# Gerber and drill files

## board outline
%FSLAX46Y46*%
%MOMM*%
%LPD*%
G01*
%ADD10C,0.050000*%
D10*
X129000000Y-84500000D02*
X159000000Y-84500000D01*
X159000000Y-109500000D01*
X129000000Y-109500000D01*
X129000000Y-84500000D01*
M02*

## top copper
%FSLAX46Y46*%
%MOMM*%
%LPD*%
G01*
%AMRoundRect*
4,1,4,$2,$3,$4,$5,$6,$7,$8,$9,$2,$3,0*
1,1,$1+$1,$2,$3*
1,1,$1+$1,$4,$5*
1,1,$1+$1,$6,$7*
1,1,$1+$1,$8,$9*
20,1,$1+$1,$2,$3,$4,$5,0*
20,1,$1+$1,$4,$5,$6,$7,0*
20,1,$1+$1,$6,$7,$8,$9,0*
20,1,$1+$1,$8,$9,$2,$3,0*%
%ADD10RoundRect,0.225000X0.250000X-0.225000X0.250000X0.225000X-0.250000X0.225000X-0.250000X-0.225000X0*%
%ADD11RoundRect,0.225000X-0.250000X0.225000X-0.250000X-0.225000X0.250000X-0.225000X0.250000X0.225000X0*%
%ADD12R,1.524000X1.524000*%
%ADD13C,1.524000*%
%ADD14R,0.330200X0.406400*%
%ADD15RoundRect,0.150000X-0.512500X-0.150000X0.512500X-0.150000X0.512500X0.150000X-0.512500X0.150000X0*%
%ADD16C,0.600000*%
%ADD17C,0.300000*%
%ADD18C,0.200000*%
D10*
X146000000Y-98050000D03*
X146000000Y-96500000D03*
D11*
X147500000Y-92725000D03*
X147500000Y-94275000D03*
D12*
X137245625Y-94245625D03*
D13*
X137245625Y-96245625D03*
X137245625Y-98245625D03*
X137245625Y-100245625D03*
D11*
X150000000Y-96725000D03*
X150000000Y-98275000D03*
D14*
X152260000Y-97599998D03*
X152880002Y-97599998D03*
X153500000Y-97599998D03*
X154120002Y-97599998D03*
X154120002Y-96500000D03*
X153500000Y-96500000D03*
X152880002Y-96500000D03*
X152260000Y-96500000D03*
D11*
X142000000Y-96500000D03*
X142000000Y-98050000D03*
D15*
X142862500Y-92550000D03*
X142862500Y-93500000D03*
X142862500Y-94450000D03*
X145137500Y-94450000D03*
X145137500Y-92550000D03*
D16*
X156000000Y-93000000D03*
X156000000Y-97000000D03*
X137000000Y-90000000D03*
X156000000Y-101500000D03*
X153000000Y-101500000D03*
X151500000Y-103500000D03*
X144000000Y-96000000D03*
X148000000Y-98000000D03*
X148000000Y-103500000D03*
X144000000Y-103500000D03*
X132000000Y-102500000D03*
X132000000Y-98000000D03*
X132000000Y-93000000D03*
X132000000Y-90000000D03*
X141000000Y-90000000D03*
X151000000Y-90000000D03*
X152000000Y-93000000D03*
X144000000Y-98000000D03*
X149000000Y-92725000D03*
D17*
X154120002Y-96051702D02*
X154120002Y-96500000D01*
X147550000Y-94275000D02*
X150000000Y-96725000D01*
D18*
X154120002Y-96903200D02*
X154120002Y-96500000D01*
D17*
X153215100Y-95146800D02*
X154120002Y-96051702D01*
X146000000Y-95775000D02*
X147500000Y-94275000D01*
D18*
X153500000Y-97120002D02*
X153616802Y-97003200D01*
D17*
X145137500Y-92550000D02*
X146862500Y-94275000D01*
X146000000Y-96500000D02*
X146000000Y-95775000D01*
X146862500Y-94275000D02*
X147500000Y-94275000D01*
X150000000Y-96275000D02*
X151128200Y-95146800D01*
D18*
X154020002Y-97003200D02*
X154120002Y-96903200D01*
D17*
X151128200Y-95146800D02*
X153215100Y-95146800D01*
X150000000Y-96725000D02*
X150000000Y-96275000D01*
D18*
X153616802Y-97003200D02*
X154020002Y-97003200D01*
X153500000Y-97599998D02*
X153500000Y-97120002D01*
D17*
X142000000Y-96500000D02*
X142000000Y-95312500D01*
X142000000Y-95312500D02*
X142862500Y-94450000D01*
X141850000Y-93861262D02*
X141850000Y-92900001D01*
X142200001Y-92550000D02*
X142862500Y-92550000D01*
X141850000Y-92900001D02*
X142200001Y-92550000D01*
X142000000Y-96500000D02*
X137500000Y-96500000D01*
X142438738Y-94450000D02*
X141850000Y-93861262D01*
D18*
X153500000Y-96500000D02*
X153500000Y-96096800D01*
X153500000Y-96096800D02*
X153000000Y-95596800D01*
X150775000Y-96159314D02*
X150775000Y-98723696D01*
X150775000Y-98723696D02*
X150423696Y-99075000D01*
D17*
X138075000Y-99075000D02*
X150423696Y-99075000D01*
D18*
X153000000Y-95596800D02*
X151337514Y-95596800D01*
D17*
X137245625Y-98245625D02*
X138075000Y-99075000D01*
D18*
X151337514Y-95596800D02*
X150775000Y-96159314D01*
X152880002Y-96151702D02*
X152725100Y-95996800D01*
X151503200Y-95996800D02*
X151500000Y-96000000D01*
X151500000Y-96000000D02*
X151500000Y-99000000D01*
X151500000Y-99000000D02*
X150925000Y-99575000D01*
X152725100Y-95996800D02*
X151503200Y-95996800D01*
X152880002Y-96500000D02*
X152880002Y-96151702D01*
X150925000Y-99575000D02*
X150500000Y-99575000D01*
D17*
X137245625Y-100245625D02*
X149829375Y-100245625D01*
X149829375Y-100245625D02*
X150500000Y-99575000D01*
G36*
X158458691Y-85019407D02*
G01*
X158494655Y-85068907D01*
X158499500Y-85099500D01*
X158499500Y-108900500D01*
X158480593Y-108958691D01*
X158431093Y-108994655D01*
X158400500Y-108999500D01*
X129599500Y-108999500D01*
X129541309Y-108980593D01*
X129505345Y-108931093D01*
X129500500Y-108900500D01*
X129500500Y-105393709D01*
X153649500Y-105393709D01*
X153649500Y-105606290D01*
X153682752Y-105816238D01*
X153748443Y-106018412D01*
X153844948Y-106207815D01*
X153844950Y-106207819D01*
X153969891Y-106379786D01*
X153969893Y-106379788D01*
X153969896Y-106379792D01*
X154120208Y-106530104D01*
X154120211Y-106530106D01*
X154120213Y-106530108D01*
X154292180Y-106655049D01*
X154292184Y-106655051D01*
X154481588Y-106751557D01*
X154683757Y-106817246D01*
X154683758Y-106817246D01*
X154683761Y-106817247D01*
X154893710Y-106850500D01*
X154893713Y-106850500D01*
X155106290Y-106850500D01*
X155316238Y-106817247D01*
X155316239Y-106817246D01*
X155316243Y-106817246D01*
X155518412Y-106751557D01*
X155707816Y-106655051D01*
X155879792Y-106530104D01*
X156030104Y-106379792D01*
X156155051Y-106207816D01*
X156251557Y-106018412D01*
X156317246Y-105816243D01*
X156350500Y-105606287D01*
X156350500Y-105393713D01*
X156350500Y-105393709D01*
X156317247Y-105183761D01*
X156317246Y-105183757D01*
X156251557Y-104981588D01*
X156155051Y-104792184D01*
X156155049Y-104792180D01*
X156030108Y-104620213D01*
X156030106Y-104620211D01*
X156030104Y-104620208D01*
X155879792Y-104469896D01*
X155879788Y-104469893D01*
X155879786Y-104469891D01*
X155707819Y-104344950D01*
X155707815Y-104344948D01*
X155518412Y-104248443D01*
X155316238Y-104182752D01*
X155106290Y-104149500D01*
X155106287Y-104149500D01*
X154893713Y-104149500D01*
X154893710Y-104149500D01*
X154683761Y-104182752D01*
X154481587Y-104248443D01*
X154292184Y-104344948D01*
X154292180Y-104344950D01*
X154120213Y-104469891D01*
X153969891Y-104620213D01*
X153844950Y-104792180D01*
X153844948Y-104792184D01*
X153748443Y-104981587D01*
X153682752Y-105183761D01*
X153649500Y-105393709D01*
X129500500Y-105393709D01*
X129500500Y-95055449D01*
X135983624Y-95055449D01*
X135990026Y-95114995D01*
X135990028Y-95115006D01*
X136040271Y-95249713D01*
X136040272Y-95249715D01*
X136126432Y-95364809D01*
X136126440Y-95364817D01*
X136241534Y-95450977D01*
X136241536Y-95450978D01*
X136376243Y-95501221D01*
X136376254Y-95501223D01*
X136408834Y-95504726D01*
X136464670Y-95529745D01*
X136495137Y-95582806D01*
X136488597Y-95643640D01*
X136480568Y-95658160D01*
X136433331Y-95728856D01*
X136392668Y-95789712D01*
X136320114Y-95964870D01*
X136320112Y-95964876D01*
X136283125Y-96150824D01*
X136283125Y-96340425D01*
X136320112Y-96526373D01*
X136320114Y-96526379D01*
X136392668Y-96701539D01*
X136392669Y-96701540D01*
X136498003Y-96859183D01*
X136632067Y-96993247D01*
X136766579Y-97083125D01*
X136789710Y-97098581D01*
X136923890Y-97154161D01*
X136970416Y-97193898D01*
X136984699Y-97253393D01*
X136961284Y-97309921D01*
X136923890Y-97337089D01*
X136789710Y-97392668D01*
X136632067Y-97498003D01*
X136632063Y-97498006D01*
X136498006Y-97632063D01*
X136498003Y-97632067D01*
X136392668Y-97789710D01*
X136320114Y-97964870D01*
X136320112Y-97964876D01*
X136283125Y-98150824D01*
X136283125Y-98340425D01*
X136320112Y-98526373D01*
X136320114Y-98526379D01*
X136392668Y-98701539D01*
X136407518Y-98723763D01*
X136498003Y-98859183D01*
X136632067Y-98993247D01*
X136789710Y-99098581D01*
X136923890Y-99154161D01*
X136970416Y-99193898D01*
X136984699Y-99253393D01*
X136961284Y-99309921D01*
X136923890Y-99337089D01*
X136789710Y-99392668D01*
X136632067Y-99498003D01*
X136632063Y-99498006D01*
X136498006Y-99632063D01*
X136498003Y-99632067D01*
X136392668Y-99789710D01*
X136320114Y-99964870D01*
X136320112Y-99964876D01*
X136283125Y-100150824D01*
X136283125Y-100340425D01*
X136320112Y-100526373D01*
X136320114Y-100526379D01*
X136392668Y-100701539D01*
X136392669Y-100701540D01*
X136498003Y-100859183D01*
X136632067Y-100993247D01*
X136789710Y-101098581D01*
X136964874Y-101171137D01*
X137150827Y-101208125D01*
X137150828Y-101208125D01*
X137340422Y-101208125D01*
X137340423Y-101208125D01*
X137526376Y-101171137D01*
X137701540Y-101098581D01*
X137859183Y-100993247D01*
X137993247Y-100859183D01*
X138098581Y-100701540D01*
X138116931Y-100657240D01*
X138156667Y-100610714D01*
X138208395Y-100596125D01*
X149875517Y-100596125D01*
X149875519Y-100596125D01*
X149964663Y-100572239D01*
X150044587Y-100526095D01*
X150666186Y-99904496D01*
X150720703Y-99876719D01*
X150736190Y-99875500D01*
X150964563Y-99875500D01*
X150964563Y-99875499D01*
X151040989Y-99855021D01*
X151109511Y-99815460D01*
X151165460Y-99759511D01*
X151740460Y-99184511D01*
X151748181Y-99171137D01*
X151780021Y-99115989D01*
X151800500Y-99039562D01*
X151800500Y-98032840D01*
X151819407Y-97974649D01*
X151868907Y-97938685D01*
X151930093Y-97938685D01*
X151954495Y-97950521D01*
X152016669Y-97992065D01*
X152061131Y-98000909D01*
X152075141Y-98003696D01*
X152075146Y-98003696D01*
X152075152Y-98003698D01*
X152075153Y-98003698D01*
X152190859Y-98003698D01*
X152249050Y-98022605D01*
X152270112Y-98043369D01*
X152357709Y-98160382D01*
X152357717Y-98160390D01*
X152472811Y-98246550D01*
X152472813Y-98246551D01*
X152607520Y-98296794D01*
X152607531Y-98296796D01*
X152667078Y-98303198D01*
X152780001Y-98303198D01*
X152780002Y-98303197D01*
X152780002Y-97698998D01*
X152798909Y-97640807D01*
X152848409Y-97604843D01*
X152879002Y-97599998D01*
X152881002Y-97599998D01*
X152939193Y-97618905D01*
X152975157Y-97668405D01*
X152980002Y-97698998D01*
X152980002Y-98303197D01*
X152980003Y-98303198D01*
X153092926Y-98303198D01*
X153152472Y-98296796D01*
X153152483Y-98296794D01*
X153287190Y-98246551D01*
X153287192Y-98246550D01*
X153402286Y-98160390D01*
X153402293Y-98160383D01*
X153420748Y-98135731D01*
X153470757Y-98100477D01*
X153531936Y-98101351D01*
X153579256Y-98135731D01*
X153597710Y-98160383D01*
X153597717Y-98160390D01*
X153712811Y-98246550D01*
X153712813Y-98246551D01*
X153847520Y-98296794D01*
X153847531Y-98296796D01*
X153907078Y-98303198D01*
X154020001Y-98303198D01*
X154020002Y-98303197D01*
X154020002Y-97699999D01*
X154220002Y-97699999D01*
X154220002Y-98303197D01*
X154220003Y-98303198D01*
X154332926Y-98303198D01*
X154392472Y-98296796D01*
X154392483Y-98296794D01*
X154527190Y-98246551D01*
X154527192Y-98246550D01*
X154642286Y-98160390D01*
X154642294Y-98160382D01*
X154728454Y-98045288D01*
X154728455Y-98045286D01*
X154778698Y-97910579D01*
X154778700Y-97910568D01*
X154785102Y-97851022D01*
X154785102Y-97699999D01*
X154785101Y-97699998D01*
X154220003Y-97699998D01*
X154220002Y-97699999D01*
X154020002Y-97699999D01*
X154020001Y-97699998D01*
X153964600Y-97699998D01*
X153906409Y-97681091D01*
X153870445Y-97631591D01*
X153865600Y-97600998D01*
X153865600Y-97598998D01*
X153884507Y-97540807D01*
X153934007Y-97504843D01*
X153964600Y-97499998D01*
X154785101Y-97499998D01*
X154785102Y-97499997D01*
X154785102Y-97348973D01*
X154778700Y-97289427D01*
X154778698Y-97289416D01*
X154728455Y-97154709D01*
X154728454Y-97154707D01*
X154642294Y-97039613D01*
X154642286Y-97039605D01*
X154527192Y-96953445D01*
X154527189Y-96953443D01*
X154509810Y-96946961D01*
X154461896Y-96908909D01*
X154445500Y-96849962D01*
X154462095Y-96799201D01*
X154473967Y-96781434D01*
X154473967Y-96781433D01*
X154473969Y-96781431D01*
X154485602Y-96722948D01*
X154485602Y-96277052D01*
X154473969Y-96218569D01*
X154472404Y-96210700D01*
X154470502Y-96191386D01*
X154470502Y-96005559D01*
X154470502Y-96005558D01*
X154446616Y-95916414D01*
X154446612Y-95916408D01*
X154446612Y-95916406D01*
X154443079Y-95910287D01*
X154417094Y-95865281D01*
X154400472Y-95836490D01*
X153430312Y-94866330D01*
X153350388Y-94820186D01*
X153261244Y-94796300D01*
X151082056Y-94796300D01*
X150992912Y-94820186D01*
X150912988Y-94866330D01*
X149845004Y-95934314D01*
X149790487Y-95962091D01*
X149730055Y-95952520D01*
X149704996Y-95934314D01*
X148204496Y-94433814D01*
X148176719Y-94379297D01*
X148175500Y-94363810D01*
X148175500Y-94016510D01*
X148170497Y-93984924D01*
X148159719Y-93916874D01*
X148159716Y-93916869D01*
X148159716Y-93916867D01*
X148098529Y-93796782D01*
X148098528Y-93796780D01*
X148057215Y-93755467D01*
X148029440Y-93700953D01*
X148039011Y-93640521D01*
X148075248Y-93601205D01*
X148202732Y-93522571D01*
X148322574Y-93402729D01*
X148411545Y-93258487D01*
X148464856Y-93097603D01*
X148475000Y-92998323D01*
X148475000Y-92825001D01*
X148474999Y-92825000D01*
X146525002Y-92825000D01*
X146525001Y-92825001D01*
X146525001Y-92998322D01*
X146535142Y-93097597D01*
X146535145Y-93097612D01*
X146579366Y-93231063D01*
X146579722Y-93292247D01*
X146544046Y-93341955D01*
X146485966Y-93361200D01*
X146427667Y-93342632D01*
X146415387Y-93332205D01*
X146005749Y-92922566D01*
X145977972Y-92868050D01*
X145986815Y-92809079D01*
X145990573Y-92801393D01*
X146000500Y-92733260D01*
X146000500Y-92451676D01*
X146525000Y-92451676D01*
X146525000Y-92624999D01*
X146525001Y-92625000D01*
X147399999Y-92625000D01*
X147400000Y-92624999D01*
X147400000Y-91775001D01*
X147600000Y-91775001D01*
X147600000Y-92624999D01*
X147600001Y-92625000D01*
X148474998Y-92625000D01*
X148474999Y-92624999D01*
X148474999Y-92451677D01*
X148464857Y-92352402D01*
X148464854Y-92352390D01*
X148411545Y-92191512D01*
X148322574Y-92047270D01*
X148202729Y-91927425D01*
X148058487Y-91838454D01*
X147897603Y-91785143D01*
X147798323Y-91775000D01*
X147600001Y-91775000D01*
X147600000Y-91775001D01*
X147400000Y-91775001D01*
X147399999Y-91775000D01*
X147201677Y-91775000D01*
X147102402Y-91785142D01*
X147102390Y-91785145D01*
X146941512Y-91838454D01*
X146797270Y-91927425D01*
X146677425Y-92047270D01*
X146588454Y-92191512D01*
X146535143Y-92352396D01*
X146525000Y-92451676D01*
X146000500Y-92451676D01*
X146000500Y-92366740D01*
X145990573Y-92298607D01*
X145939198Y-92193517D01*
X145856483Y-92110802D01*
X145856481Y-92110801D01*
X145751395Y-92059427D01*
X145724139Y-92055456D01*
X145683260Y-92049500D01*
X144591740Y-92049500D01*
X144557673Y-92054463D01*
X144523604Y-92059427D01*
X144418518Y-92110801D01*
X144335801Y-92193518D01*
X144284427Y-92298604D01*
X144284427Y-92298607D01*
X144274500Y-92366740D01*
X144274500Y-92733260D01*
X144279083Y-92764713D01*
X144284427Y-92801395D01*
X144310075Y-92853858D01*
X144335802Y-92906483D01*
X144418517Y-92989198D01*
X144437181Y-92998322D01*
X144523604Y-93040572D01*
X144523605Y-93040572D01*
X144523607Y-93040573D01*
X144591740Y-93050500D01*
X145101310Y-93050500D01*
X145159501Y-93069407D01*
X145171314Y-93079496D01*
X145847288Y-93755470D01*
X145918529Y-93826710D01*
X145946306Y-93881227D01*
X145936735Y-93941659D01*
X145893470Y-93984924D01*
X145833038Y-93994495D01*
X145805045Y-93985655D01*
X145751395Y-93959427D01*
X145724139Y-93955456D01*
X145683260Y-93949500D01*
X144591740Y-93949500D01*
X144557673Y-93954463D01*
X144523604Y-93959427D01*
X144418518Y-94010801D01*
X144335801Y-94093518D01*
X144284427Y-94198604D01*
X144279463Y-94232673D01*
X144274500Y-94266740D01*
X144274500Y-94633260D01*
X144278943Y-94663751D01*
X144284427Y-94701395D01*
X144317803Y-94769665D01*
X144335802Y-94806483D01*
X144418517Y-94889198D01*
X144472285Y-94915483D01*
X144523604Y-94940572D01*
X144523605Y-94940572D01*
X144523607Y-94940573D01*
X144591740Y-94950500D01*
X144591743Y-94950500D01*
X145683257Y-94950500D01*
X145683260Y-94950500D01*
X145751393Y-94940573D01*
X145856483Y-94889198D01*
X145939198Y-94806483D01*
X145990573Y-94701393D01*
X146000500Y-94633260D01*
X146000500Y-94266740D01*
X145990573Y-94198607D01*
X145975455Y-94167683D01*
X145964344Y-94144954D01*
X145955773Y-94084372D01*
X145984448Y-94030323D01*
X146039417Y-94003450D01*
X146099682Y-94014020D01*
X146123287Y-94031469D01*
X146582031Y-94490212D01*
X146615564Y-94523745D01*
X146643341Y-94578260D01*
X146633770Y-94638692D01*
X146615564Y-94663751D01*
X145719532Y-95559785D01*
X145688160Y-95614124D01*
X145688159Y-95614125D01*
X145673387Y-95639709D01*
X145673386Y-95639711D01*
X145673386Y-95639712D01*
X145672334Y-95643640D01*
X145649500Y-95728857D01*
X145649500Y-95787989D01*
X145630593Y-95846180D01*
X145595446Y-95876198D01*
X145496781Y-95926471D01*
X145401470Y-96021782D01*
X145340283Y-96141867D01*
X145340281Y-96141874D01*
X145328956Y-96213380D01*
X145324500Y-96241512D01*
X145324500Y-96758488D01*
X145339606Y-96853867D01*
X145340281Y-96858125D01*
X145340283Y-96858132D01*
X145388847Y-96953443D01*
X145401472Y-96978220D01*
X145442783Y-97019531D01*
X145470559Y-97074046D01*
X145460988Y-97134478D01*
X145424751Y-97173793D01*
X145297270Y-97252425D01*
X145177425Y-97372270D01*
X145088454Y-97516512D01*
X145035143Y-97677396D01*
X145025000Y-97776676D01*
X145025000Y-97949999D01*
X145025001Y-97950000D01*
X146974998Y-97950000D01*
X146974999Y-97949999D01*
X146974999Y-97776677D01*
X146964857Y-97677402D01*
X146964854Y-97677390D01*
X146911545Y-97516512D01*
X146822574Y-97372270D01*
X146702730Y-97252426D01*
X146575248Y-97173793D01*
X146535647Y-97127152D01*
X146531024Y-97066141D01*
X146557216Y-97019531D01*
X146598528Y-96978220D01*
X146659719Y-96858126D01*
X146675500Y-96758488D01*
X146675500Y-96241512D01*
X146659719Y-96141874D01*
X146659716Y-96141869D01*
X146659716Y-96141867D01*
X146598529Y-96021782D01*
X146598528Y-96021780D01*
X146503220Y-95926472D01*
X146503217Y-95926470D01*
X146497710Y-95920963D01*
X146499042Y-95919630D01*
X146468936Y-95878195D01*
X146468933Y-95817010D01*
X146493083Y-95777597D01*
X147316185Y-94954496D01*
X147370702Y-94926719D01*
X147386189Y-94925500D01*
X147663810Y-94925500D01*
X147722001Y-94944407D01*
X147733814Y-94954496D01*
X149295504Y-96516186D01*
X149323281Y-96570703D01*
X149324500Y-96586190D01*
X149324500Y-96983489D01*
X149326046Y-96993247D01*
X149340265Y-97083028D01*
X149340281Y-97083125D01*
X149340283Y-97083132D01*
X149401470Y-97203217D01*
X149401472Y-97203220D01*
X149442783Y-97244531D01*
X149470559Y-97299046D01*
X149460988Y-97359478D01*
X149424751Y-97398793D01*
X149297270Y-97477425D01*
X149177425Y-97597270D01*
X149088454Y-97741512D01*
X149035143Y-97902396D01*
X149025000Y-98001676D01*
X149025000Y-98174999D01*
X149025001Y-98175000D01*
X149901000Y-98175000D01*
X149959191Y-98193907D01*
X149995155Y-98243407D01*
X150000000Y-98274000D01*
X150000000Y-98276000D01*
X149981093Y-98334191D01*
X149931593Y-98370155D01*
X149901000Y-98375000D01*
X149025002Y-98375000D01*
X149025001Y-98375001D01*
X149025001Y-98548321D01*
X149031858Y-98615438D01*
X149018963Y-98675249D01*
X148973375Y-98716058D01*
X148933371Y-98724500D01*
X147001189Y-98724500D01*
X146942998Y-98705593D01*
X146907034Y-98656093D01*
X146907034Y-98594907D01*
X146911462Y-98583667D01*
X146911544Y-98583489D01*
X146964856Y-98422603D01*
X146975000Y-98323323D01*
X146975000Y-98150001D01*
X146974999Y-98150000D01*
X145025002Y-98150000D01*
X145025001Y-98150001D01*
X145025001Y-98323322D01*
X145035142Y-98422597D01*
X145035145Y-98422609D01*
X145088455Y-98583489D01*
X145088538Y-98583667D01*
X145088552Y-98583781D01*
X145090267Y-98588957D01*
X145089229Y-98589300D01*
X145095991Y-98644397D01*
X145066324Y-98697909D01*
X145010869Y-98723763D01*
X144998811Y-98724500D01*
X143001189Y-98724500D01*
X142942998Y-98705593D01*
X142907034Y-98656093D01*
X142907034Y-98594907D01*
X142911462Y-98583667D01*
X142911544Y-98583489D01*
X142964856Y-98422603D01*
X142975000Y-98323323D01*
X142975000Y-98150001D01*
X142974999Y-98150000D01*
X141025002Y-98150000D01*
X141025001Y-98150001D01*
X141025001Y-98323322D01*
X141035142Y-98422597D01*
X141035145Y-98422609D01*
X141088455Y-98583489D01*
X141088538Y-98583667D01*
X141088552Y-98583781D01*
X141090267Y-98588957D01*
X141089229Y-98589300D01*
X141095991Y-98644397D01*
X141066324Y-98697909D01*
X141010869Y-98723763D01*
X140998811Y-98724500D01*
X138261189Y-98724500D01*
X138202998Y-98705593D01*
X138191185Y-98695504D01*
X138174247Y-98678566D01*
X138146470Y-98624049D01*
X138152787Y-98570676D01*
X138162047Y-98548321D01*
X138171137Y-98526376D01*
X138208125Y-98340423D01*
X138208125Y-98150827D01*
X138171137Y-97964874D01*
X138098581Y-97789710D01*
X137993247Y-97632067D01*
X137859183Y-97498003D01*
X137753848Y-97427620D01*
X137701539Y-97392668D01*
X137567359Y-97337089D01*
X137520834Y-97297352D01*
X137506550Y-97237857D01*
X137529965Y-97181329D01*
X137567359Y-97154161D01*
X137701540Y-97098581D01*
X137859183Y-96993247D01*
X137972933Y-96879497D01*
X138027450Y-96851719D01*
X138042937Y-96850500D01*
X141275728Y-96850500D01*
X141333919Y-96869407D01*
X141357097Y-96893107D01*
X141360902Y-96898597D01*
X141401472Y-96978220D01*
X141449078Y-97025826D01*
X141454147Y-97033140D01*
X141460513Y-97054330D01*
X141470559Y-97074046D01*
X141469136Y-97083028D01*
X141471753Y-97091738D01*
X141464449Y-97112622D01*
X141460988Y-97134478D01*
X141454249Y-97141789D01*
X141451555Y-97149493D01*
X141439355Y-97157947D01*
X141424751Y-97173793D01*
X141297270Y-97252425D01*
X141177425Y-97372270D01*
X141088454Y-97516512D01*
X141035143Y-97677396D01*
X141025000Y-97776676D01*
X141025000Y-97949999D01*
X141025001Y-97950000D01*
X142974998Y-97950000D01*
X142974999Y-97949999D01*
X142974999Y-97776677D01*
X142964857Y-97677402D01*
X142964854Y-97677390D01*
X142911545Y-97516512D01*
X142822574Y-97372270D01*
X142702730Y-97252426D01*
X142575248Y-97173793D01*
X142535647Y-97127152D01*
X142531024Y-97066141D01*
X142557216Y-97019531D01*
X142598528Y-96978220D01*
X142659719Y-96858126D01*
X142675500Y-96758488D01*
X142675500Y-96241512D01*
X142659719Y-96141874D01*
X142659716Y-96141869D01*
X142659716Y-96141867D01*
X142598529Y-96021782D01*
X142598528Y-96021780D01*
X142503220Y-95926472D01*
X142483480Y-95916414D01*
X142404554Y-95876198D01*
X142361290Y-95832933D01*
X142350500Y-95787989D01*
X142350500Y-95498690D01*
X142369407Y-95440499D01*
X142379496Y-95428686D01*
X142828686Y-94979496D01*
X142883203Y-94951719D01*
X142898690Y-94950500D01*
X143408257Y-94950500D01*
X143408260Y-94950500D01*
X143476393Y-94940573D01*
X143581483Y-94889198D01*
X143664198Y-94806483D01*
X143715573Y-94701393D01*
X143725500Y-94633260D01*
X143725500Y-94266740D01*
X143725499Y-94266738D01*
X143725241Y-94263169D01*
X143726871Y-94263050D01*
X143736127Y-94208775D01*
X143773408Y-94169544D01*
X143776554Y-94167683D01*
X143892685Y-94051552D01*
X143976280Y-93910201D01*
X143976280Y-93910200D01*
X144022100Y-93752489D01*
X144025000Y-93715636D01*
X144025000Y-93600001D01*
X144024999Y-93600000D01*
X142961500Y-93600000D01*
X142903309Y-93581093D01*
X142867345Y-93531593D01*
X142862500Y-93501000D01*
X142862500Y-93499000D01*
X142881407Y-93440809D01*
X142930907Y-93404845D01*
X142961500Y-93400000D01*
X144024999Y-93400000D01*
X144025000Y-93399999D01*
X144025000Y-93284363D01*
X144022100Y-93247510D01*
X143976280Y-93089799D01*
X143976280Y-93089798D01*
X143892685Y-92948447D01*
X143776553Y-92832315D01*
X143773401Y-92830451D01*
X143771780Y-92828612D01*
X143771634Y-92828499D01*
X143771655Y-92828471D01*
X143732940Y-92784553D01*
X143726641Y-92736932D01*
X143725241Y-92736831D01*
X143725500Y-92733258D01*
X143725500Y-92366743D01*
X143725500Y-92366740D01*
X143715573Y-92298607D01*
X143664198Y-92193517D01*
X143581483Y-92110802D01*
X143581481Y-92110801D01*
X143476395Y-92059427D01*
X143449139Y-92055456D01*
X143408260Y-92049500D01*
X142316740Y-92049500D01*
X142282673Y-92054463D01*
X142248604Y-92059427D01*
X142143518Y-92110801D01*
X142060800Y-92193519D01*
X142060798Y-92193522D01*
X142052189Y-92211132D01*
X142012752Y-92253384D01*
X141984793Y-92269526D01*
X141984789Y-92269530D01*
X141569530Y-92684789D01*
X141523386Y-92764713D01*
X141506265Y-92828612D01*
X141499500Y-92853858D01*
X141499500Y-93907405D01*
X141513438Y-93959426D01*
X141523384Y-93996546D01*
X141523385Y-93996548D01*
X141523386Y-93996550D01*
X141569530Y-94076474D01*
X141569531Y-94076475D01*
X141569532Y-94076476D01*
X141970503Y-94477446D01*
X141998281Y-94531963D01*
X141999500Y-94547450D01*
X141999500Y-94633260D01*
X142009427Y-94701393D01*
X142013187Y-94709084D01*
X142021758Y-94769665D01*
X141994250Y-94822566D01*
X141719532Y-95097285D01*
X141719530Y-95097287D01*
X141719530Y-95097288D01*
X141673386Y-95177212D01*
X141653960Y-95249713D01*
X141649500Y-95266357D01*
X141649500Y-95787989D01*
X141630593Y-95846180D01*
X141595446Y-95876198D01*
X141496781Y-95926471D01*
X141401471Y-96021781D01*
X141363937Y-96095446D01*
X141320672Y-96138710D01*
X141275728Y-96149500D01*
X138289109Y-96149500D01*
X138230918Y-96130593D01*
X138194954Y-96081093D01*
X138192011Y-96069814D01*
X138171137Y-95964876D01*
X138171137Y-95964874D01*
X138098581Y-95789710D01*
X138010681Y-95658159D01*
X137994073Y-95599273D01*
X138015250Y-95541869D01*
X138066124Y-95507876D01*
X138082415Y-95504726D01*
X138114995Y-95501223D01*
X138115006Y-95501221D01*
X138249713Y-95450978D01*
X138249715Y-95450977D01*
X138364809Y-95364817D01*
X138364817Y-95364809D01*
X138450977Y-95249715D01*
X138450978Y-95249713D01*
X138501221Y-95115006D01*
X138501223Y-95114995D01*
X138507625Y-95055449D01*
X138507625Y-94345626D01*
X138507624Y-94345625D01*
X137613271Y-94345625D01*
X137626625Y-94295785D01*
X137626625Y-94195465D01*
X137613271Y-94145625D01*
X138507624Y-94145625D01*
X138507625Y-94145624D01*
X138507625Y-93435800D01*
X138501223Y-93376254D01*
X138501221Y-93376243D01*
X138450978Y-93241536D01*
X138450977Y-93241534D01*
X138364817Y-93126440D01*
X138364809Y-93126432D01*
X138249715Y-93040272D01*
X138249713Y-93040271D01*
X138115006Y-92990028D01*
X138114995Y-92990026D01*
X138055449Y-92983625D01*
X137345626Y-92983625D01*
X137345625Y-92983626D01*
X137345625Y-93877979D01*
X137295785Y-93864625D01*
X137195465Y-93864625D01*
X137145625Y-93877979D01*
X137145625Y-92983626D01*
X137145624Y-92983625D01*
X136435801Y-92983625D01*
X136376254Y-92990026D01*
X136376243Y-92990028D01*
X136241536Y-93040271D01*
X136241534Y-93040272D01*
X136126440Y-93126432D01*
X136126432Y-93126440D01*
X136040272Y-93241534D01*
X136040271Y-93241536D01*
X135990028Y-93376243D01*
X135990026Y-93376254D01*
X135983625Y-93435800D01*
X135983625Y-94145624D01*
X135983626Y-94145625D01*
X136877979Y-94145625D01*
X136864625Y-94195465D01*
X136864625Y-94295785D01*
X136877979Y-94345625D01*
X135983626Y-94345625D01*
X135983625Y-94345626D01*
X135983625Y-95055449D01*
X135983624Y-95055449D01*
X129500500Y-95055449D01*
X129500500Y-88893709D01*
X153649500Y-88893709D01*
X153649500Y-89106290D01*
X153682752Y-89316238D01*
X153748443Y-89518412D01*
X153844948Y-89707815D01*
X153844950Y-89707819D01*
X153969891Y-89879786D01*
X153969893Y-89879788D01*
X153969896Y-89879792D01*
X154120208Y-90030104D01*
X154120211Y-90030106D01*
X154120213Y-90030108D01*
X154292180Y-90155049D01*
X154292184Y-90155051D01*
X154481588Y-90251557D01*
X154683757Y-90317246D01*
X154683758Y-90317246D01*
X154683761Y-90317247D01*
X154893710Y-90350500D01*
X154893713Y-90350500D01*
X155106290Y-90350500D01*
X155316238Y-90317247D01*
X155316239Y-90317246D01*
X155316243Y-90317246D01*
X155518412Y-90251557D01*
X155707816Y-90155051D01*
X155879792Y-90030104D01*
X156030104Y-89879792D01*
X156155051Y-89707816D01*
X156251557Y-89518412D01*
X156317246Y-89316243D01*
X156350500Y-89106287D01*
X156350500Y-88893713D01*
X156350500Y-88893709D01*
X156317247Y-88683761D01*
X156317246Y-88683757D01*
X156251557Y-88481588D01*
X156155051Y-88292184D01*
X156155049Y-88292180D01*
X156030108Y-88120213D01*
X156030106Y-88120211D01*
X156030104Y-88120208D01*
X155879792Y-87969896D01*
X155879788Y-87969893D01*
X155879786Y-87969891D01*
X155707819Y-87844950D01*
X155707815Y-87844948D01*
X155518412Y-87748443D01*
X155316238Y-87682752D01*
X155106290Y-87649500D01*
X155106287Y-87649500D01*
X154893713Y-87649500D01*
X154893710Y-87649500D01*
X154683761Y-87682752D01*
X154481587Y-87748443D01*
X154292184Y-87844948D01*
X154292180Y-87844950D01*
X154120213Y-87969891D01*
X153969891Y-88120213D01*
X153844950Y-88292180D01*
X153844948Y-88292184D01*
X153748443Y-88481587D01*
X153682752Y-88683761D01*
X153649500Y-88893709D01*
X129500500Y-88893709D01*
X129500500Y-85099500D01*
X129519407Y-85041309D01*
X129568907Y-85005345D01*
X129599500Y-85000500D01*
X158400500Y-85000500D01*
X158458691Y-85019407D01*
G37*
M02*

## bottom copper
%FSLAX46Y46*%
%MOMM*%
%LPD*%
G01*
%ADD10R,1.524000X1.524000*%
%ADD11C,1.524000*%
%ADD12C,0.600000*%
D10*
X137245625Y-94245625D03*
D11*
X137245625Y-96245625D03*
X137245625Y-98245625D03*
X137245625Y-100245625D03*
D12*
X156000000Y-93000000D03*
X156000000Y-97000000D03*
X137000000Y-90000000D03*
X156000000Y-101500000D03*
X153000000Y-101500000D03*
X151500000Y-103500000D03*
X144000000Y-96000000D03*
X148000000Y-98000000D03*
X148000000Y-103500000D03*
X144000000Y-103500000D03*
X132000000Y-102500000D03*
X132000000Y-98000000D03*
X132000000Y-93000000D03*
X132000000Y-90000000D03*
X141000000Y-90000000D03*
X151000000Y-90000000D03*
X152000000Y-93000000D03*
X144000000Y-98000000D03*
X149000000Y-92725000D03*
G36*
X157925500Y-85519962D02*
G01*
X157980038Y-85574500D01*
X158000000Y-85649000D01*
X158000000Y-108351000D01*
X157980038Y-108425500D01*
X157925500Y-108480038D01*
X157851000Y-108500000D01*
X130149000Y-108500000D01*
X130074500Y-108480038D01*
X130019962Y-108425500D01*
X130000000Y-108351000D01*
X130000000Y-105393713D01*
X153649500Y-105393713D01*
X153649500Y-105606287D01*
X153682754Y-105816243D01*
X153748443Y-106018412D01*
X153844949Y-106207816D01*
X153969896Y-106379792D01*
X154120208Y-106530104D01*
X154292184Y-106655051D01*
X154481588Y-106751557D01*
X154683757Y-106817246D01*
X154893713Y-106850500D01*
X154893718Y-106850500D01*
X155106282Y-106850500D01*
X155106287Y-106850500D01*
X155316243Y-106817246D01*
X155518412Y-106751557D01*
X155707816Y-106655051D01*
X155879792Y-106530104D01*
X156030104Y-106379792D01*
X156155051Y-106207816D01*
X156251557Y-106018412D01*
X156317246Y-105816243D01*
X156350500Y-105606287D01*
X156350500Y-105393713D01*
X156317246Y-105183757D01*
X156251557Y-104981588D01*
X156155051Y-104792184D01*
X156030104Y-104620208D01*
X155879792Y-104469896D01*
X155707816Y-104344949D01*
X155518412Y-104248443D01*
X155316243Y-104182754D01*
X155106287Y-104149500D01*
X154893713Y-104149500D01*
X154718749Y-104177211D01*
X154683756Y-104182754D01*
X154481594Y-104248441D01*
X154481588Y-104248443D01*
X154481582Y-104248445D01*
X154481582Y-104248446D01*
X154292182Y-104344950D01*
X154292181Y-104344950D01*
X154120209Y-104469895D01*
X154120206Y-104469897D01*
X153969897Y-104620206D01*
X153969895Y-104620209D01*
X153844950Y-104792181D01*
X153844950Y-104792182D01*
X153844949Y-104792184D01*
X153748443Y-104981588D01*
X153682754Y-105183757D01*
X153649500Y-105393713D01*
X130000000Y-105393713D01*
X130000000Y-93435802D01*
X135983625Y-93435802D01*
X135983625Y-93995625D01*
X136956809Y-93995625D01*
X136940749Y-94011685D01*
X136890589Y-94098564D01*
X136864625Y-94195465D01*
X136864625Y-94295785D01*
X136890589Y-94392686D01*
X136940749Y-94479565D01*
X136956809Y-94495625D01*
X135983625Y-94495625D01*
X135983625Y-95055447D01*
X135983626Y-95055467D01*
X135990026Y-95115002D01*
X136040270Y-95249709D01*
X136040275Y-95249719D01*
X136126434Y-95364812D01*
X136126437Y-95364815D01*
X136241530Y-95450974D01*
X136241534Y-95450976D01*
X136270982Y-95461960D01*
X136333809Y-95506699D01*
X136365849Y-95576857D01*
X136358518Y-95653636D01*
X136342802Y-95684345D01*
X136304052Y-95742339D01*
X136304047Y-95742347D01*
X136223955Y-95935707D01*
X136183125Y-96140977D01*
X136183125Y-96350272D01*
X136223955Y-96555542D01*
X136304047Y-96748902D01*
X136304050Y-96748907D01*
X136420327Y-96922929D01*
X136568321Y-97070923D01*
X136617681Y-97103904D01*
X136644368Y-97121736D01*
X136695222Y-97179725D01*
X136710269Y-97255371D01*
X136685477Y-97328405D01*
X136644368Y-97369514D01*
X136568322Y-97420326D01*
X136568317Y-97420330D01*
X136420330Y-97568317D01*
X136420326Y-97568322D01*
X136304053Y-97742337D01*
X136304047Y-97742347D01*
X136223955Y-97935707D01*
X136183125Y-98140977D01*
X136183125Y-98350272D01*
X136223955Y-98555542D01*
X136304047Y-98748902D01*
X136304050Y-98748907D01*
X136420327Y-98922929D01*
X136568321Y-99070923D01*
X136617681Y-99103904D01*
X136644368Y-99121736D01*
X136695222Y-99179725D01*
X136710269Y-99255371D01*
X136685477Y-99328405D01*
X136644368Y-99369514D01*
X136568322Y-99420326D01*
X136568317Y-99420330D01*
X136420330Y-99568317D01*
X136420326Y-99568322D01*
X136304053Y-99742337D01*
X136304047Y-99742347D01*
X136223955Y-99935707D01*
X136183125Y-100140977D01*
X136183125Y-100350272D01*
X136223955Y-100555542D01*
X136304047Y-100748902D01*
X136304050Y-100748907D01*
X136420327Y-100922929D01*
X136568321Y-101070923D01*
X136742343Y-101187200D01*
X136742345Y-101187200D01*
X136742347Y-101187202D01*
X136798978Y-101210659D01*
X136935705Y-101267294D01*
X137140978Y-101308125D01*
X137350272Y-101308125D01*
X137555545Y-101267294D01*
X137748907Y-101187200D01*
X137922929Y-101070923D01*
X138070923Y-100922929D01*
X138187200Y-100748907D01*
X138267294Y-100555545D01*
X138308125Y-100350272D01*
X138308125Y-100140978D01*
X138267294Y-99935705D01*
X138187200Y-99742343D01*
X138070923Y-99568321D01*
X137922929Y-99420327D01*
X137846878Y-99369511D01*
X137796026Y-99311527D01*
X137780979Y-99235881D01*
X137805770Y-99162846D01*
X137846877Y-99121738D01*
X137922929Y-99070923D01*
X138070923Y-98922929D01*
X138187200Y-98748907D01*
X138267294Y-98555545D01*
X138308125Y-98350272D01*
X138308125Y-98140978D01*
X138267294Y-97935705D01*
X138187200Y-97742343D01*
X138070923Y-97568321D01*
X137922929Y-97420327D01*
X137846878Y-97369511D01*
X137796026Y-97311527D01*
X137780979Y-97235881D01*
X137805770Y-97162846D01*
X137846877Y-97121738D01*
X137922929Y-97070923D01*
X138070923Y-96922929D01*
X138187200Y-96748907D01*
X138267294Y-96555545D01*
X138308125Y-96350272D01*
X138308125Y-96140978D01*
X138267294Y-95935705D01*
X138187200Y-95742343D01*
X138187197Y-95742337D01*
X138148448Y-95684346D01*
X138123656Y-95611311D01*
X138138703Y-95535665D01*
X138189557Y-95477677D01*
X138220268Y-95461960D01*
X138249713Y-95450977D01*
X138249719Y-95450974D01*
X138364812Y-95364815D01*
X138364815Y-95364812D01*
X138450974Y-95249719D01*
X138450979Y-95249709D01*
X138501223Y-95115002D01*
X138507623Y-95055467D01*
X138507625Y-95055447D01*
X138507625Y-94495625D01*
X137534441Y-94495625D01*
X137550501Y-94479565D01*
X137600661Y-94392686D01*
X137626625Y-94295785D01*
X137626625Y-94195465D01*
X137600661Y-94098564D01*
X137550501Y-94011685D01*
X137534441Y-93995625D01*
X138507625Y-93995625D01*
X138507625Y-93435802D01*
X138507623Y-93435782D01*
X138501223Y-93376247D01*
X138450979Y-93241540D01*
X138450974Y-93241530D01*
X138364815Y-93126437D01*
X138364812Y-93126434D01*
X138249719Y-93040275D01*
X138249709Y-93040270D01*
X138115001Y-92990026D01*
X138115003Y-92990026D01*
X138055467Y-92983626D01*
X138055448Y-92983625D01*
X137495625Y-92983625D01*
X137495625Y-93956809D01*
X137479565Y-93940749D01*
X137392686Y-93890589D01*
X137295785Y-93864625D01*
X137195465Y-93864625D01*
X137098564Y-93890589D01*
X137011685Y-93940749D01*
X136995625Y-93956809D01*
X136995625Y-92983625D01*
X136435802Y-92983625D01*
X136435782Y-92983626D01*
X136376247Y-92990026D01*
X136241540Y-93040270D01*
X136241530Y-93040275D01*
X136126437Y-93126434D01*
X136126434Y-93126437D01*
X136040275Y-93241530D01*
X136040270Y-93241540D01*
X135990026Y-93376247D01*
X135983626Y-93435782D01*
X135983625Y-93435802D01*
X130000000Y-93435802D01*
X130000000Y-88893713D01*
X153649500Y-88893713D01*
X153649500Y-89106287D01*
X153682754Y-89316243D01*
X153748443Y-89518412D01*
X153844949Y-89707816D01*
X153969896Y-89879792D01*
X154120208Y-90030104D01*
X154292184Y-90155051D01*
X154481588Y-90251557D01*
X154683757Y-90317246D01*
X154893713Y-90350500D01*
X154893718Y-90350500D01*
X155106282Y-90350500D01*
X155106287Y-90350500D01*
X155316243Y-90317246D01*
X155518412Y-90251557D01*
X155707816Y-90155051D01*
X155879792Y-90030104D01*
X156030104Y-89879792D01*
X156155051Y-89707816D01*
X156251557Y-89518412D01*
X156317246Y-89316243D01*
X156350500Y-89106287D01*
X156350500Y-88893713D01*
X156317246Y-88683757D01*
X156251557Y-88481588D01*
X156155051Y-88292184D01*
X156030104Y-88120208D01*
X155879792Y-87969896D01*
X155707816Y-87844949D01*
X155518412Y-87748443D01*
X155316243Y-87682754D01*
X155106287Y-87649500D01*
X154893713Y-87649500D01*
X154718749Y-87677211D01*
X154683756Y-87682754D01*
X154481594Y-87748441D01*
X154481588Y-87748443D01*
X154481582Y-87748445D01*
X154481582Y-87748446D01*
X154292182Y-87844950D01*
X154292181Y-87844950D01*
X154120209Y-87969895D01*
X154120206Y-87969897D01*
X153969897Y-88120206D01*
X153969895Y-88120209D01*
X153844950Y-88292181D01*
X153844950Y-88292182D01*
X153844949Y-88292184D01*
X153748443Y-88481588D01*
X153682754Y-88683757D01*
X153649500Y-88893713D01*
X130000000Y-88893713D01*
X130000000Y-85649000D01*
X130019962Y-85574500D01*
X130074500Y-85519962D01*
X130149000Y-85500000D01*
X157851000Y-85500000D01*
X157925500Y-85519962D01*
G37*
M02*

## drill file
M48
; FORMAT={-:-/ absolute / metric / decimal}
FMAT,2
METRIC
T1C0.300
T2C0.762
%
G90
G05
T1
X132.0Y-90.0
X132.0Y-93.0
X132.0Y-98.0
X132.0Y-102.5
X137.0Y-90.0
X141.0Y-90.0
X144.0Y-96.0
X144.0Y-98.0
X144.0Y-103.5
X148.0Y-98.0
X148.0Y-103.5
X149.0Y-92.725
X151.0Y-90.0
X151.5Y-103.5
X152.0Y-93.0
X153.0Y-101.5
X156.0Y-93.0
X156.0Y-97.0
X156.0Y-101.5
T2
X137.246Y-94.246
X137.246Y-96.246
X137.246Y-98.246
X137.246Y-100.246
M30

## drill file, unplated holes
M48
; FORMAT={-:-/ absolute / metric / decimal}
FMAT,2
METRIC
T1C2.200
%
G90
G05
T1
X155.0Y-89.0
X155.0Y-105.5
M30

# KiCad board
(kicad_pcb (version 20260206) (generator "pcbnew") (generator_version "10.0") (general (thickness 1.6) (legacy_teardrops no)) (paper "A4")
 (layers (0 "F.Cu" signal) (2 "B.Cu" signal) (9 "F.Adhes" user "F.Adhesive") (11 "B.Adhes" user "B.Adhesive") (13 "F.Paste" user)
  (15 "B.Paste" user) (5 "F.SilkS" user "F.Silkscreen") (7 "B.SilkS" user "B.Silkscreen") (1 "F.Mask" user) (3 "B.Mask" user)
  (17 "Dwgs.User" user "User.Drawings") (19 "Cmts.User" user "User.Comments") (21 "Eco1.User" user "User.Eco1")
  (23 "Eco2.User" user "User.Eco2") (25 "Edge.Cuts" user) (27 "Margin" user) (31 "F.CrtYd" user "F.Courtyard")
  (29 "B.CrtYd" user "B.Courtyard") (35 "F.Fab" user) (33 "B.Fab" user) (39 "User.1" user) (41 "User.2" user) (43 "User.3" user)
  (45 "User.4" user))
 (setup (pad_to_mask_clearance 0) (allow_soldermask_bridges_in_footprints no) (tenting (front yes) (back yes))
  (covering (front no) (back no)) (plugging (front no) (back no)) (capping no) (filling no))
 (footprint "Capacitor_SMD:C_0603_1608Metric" (layer "F.Cu") (at 146 97.275 90)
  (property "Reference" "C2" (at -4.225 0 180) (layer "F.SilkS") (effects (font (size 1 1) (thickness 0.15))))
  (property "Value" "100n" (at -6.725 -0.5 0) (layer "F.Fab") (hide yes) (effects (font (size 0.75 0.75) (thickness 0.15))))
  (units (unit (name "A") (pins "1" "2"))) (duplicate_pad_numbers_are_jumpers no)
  (pad "1" smd roundrect (at -0.775 0 90) (size 0.9 0.95) (layers "F.Cu" "F.Mask" "F.Paste") (roundrect_rratio 0.25) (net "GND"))
  (pad "2" smd roundrect (at 0.775 0 90) (size 0.9 0.95) (layers "F.Cu" "F.Mask" "F.Paste") (roundrect_rratio 0.25) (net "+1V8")))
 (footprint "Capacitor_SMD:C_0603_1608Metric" (layer "F.Cu") (at 147.5 93.5 -90)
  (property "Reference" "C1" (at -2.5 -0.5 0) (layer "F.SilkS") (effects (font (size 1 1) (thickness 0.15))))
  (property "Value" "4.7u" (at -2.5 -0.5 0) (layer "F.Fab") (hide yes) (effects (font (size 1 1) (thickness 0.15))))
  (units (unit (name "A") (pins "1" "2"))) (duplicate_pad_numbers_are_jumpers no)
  (pad "1" smd roundrect (at -0.775 0 270) (size 0.9 0.95) (layers "F.Cu" "F.Mask" "F.Paste") (roundrect_rratio 0.25) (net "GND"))
  (pad "2" smd roundrect (at 0.775 0 270) (size 0.9 0.95) (layers "F.Cu" "F.Mask" "F.Paste") (roundrect_rratio 0.25) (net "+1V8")))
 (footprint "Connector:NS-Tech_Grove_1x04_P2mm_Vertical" (layer "F.Cu") (at 137.245625 94.245625)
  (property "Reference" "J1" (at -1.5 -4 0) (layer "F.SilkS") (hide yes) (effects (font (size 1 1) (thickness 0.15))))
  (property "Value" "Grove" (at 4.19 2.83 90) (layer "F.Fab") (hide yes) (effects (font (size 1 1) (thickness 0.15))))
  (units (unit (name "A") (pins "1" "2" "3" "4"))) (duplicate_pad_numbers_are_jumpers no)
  (pad "1" thru_hole rect (at 0 0) (size 1.524 1.524) (drill 0.762) (layers "*.Cu" "*.Mask") (remove_unused_layers no) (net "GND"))
  (pad "2" thru_hole circle (at 0 2) (size 1.524 1.524) (drill 0.762) (layers "*.Cu" "*.Mask") (remove_unused_layers no) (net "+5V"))
  (pad "3" thru_hole circle (at 0 4) (size 1.524 1.524) (drill 0.762) (layers "*.Cu" "*.Mask") (remove_unused_layers no) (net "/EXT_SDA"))
  (pad "4" thru_hole circle (at 0 6) (size 1.524 1.524) (drill 0.762) (layers "*.Cu" "*.Mask") (remove_unused_layers no) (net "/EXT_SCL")))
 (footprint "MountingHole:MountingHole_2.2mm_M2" (layer "F.Cu") (at 155 105.5)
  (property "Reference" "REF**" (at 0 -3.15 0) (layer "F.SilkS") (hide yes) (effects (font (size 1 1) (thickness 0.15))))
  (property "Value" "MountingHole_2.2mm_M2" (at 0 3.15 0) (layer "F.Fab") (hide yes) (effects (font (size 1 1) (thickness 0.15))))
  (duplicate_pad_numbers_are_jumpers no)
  (pad "" np_thru_hole circle (at 0 0) (size 2.2 2.2) (drill 2.2) (layers "*.Cu" "*.Mask")))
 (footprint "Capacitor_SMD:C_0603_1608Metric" (layer "F.Cu") (at 150 97.5 -90)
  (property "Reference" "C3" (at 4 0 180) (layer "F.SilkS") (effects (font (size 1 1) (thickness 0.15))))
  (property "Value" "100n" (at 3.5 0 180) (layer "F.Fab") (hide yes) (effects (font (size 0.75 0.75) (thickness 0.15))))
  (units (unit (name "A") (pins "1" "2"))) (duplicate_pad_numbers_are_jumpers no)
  (pad "1" smd roundrect (at -0.775 0 270) (size 0.9 0.95) (layers "F.Cu" "F.Mask" "F.Paste") (roundrect_rratio 0.25) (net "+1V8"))
  (pad "2" smd roundrect (at 0.775 0 270) (size 0.9 0.95) (layers "F.Cu" "F.Mask" "F.Paste") (roundrect_rratio 0.25) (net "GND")))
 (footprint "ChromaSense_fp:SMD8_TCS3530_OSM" (layer "F.Cu") (at 153.190001 97.049999 90)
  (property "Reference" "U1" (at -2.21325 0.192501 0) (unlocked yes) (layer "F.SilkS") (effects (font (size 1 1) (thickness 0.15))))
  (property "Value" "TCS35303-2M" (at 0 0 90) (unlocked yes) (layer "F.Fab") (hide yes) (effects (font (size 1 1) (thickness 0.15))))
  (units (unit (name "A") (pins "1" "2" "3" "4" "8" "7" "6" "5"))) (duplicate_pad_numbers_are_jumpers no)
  (pad "1" smd rect (at -0.549999 -0.930001 90) (size 0.4064 0.3302) (layers "F.Cu" "F.Mask" "F.Paste") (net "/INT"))
  (pad "2" smd rect (at -0.549999 -0.309999 90) (size 0.4064 0.3302) (layers "F.Cu" "F.Mask" "F.Paste") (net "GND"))
  (pad "3" smd rect (at -0.549999 0.309999 90) (size 0.4064 0.3302) (layers "F.Cu" "F.Mask" "F.Paste") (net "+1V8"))
  (pad "4" smd rect (at -0.549999 0.930001 90) (size 0.4064 0.3302) (layers "F.Cu" "F.Mask" "F.Paste") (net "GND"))
  (pad "5" smd rect (at 0.549999 0.930001 90) (size 0.4064 0.3302) (layers "F.Cu" "F.Mask" "F.Paste") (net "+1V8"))
  (pad "6" smd rect (at 0.549999 0.309999 90) (size 0.4064 0.3302) (layers "F.Cu" "F.Mask" "F.Paste") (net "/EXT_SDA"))
  (pad "7" smd rect (at 0.549999 -0.309999 90) (size 0.4064 0.3302) (layers "F.Cu" "F.Mask" "F.Paste") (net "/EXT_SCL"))
  (pad "8" smd rect (at 0.549999 -0.930001 90) (size 0.4064 0.3302) (layers "F.Cu" "F.Mask" "F.Paste")
   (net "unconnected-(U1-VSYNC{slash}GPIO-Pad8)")))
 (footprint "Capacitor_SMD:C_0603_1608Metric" (layer "F.Cu") (at 142 97.275 -90)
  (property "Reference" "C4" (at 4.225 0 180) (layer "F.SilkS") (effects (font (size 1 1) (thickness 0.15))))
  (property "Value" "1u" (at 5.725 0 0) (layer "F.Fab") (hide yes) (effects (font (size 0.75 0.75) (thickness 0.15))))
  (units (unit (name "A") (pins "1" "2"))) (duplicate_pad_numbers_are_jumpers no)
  (pad "1" smd roundrect (at -0.775 0 270) (size 0.9 0.95) (layers "F.Cu" "F.Mask" "F.Paste") (roundrect_rratio 0.25) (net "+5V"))
  (pad "2" smd roundrect (at 0.775 0 270) (size 0.9 0.95) (layers "F.Cu" "F.Mask" "F.Paste") (roundrect_rratio 0.25) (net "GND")))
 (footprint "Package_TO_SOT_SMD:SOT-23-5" (layer "F.Cu") (at 144 93.5)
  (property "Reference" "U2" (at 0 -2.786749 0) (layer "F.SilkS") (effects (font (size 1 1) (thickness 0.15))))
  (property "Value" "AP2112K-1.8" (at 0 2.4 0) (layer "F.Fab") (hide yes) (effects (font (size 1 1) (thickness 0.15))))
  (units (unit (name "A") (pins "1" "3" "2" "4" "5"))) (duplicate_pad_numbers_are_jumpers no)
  (pad "1" smd roundrect (at -1.1375 -0.95) (size 1.325 0.6) (layers "F.Cu" "F.Mask" "F.Paste") (roundrect_rratio 0.25) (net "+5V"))
  (pad "2" smd roundrect (at -1.1375 0) (size 1.325 0.6) (layers "F.Cu" "F.Mask" "F.Paste") (roundrect_rratio 0.25) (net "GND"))
  (pad "3" smd roundrect (at -1.1375 0.95) (size 1.325 0.6) (layers "F.Cu" "F.Mask" "F.Paste") (roundrect_rratio 0.25) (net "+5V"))
  (pad "4" smd roundrect (at 1.1375 0.95) (size 1.325 0.6) (layers "F.Cu" "F.Mask" "F.Paste") (roundrect_rratio 0.25)
   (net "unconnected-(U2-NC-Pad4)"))
  (pad "5" smd roundrect (at 1.1375 -0.95) (size 1.325 0.6) (layers "F.Cu" "F.Mask" "F.Paste") (roundrect_rratio 0.25) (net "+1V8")))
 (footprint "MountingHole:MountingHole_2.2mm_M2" (layer "F.Cu") (at 155 89)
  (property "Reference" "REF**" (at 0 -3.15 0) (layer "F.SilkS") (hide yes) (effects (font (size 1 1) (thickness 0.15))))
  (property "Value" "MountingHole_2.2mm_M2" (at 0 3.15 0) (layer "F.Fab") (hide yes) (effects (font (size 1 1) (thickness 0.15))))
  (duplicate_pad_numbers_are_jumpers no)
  (pad "" np_thru_hole circle (at 0 0) (size 2.2 2.2) (drill 2.2) (layers "*.Cu" "*.Mask")))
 (gr_rect (start 129 84.5) (end 159 109.5) (stroke (width 0.05) (type solid)) (fill no) (layer "Edge.Cuts"))
 (via (at 156 93) (size 0.6) (drill 0.3) (layers "F.Cu" "B.Cu") (free yes) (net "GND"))
 (via (at 144 96) (size 0.6) (drill 0.3) (layers "F.Cu" "B.Cu") (free yes) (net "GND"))
 (via (at 151 90) (size 0.6) (drill 0.3) (layers "F.Cu" "B.Cu") (free yes) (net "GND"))
 (via (at 152 93) (size 0.6) (drill 0.3) (layers "F.Cu" "B.Cu") (free yes) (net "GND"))
 (via (at 148 98) (size 0.6) (drill 0.3) (layers "F.Cu" "B.Cu") (free yes) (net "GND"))
 (via (at 156 101.5) (size 0.6) (drill 0.3) (layers "F.Cu" "B.Cu") (free yes) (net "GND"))
 (via (at 148 103.5) (size 0.6) (drill 0.3) (layers "F.Cu" "B.Cu") (free yes) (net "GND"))
 (via (at 132 90) (size 0.6) (drill 0.3) (layers "F.Cu" "B.Cu") (free yes) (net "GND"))
 (via (at 132 102.5) (size 0.6) (drill 0.3) (layers "F.Cu" "B.Cu") (free yes) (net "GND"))
 (via (at 153 101.5) (size 0.6) (drill 0.3) (layers "F.Cu" "B.Cu") (free yes) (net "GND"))
 (via (at 132 93) (size 0.6) (drill 0.3) (layers "F.Cu" "B.Cu") (free yes) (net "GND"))
 (via (at 144 98) (size 0.6) (drill 0.3) (layers "F.Cu" "B.Cu") (free yes) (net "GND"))
 (via (at 141 90) (size 0.6) (drill 0.3) (layers "F.Cu" "B.Cu") (free yes) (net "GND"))
 (via (at 151.5 103.5) (size 0.6) (drill 0.3) (layers "F.Cu" "B.Cu") (free yes) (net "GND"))
 (via (at 149 92.725) (size 0.6) (drill 0.3) (layers "F.Cu" "B.Cu") (free yes) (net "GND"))
 (via (at 144 103.5) (size 0.6) (drill 0.3) (layers "F.Cu" "B.Cu") (free yes) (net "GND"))
 (via (at 137 90) (size 0.6) (drill 0.3) (layers "F.Cu" "B.Cu") (free yes) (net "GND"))
 (via (at 132 98) (size 0.6) (drill 0.3) (layers "F.Cu" "B.Cu") (free yes) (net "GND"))
 (via (at 156 97) (size 0.6) (drill 0.3) (layers "F.Cu" "B.Cu") (free yes) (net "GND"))
 (segment (start 154.120002 96.051702) (end 154.120002 96.5) (width 0.3) (layer "F.Cu") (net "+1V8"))
 (segment (start 147.55 94.275) (end 150 96.725) (width 0.3) (layer "F.Cu") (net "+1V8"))
 (segment (start 154.120002 96.9032) (end 154.120002 96.5) (width 0.2) (layer "F.Cu") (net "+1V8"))
 (segment (start 153.2151 95.1468) (end 154.120002 96.051702) (width 0.3) (layer "F.Cu") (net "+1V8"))
 (segment (start 146 95.775) (end 147.5 94.275) (width 0.3) (layer "F.Cu") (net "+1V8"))
 (segment (start 153.5 97.120002) (end 153.616802 97.0032) (width 0.2) (layer "F.Cu") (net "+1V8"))
 (segment (start 145.1375 92.55) (end 146.8625 94.275) (width 0.3) (layer "F.Cu") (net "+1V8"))
 (segment (start 146 96.5) (end 146 95.775) (width 0.3) (layer "F.Cu") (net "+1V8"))
 (segment (start 146.8625 94.275) (end 147.5 94.275) (width 0.3) (layer "F.Cu") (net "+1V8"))
 (segment (start 150 96.275) (end 151.1282 95.1468) (width 0.3) (layer "F.Cu") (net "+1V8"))
 (segment (start 154.020002 97.0032) (end 154.120002 96.9032) (width 0.2) (layer "F.Cu") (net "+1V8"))
 (segment (start 151.1282 95.1468) (end 153.2151 95.1468) (width 0.3) (layer "F.Cu") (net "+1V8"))
 (segment (start 150 96.725) (end 150 96.275) (width 0.3) (layer "F.Cu") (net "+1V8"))
 (segment (start 153.616802 97.0032) (end 154.020002 97.0032) (width 0.2) (layer "F.Cu") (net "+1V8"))
 (segment (start 153.5 97.599998) (end 153.5 97.120002) (width 0.2) (layer "F.Cu") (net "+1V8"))
 (segment (start 142 96.5) (end 142 95.3125) (width 0.3) (layer "F.Cu") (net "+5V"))
 (segment (start 142 95.3125) (end 142.8625 94.45) (width 0.3) (layer "F.Cu") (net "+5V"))
 (segment (start 141.85 93.861262) (end 141.85 92.900001) (width 0.3) (layer "F.Cu") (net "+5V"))
 (segment (start 142.200001 92.55) (end 142.8625 92.55) (width 0.3) (layer "F.Cu") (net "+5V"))
 (segment (start 141.85 92.900001) (end 142.200001 92.55) (width 0.3) (layer "F.Cu") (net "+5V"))
 (segment (start 142 96.5) (end 137.5 96.5) (width 0.3) (layer "F.Cu") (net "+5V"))
 (segment (start 142.438738 94.45) (end 141.85 93.861262) (width 0.3) (layer "F.Cu") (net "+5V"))
 (segment (start 153.5 96.5) (end 153.5 96.0968) (width 0.2) (layer "F.Cu") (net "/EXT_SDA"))
 (segment (start 153.5 96.0968) (end 153 95.5968) (width 0.2) (layer "F.Cu") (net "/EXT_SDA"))
 (segment (start 150.775 96.159314) (end 150.775 98.723696) (width 0.2) (layer "F.Cu") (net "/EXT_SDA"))
 (segment (start 150.775 98.723696) (end 150.423696 99.075) (width 0.2) (layer "F.Cu") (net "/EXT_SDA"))
 (segment (start 138.075 99.075) (end 150.423696 99.075) (width 0.3) (layer "F.Cu") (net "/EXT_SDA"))
 (segment (start 153 95.5968) (end 151.337514 95.5968) (width 0.2) (layer "F.Cu") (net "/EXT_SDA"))
 (segment (start 137.245625 98.245625) (end 138.075 99.075) (width 0.3) (layer "F.Cu") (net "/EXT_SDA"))
 (segment (start 151.337514 95.5968) (end 150.775 96.159314) (width 0.2) (layer "F.Cu") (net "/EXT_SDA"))
 (segment (start 152.880002 96.151702) (end 152.7251 95.9968) (width 0.2) (layer "F.Cu") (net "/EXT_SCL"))
 (segment (start 151.5032 95.9968) (end 151.5 96) (width 0.2) (layer "F.Cu") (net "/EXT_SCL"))
 (segment (start 151.5 96) (end 151.5 99) (width 0.2) (layer "F.Cu") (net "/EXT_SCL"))
 (segment (start 151.5 99) (end 150.925 99.575) (width 0.2) (layer "F.Cu") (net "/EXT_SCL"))
 (segment (start 152.7251 95.9968) (end 151.5032 95.9968) (width 0.2) (layer "F.Cu") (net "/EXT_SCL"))
 (segment (start 152.880002 96.5) (end 152.880002 96.151702) (width 0.2) (layer "F.Cu") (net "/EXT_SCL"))
 (segment (start 150.925 99.575) (end 150.5 99.575) (width 0.2) (layer "F.Cu") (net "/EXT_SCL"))
 (segment (start 137.245625 100.245625) (end 149.829375 100.245625) (width 0.3) (layer "F.Cu") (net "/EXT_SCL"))
 (segment (start 149.829375 100.245625) (end 150.5 99.575) (width 0.3) (layer "F.Cu") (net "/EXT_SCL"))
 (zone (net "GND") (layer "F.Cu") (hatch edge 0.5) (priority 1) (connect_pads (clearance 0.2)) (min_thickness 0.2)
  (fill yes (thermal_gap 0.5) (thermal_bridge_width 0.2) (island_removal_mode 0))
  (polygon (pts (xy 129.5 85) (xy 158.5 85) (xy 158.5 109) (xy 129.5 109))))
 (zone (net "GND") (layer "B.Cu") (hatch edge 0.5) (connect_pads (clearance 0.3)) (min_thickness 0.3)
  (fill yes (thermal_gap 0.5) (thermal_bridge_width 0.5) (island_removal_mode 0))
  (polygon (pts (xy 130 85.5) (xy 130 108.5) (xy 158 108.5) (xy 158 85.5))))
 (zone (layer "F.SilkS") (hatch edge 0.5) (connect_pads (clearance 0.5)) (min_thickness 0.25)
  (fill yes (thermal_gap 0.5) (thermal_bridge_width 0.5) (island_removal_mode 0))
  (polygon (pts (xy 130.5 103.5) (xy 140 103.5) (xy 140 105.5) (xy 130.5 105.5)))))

